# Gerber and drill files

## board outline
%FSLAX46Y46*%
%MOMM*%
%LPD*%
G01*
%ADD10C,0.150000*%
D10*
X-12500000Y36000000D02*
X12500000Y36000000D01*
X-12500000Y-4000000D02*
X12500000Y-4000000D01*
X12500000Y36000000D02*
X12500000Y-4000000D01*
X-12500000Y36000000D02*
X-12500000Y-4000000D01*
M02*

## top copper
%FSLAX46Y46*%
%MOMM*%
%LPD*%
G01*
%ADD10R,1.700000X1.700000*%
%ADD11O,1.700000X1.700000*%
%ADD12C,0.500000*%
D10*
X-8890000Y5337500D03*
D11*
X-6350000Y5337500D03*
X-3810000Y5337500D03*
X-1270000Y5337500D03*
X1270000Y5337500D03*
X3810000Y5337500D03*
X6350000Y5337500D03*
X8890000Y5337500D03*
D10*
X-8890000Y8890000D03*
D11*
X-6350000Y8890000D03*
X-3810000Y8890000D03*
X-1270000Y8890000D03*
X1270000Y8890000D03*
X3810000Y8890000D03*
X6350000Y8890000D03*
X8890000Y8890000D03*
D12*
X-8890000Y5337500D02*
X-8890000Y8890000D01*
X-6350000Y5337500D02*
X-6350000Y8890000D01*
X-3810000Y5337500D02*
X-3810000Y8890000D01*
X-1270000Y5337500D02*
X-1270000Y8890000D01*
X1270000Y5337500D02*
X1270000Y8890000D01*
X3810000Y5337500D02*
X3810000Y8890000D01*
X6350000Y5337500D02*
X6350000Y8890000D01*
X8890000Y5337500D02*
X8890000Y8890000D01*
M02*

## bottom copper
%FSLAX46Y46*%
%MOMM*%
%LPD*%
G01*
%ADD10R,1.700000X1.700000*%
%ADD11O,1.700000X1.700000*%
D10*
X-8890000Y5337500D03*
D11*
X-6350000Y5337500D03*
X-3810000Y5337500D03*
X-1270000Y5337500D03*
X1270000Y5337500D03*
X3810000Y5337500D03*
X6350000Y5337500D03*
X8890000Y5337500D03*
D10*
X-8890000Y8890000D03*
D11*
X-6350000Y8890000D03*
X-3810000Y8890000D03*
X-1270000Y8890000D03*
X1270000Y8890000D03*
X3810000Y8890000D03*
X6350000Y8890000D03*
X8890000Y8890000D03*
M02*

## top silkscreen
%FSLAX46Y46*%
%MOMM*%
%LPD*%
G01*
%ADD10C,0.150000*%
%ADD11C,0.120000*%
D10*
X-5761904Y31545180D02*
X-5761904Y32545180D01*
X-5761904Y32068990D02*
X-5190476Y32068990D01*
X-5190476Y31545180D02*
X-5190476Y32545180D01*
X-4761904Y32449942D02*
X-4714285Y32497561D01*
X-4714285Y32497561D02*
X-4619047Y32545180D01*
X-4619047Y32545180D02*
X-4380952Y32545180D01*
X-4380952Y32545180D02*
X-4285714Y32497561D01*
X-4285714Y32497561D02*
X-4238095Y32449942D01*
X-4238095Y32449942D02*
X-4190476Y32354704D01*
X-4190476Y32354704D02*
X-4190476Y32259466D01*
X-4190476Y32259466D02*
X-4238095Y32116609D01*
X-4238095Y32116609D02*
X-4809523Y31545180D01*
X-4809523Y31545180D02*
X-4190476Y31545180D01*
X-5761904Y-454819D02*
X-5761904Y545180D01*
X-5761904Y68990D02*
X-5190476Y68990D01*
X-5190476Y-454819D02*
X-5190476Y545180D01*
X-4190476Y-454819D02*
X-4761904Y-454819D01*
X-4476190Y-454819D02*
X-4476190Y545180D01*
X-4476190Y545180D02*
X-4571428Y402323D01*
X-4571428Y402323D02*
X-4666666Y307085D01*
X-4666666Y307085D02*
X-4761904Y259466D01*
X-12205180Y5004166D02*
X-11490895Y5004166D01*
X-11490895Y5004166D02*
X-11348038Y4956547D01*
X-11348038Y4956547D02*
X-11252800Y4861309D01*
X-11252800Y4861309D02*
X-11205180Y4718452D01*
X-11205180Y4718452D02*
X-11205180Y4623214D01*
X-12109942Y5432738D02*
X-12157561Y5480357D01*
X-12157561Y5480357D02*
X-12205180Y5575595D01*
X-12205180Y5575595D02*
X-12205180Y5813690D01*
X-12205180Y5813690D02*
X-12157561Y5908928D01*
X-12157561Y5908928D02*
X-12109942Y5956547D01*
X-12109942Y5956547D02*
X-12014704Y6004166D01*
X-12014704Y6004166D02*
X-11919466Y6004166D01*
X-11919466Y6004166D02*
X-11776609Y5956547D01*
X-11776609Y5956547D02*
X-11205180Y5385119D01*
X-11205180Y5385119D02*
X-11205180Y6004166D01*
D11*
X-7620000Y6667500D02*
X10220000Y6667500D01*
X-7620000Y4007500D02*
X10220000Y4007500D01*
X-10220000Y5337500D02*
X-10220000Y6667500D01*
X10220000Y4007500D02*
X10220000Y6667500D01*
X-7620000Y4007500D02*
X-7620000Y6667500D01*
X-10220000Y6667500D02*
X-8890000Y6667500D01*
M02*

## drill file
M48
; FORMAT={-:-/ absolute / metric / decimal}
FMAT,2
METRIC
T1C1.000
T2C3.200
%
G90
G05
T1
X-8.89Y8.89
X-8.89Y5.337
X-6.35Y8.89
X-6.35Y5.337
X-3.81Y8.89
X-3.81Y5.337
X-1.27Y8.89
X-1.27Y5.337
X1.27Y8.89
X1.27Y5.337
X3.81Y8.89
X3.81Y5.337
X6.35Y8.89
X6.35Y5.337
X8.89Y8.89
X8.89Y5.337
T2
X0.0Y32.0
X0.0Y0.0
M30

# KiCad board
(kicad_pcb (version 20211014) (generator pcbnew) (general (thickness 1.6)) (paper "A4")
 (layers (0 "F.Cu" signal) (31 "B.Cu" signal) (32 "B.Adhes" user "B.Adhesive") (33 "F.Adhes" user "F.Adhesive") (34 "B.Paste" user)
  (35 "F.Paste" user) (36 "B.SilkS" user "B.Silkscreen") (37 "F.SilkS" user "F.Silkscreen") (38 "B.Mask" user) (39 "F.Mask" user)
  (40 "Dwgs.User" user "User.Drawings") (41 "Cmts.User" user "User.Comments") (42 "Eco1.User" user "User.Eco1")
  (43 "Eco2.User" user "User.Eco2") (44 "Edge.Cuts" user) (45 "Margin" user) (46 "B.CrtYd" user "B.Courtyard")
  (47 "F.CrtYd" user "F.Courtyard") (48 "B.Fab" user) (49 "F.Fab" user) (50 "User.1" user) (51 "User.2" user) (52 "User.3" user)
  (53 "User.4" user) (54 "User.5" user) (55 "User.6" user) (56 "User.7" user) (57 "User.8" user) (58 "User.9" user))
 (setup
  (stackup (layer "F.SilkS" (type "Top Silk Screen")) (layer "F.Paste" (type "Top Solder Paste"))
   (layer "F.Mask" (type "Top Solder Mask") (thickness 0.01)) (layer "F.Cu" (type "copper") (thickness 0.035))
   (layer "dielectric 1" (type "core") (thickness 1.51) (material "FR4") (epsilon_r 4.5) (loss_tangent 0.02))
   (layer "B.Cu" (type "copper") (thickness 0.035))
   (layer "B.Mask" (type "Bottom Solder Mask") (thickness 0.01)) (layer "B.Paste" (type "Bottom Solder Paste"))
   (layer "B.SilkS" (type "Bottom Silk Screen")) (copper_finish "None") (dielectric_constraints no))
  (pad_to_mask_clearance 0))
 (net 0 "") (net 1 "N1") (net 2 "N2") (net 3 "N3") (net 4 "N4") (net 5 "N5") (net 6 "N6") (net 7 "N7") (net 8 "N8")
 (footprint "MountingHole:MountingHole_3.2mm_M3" (layer "F.Cu") (at 0 -32)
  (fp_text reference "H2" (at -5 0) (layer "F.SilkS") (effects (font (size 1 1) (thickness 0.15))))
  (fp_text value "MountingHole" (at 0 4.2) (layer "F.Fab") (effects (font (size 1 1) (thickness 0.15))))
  (pad "" np_thru_hole circle (at 0 0) (size 3.2 3.2) (drill 3.2) (layers *.Cu *.Mask)))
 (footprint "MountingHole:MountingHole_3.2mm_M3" (layer "F.Cu") (at 0 0)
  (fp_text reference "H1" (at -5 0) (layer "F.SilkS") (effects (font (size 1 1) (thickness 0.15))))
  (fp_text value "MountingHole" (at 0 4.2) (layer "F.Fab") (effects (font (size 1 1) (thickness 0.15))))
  (pad "" np_thru_hole circle (at 0 0) (size 3.2 3.2) (drill 3.2) (layers *.Cu *.Mask)))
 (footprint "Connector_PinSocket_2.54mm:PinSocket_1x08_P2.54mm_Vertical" (layer "F.Cu") (at -8.89 -5.3375 90)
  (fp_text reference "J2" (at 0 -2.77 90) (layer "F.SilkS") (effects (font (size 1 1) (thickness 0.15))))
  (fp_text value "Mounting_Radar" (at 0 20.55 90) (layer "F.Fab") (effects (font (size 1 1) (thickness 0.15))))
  (fp_line (start 1.33 1.27) (end 1.33 19.11) (layer "F.SilkS") (width 0.12))
  (fp_line (start -1.33 1.27) (end -1.33 19.11) (layer "F.SilkS") (width 0.12))
  (fp_line (start 0 -1.33) (end 1.33 -1.33) (layer "F.SilkS") (width 0.12))
  (fp_line (start -1.33 19.11) (end 1.33 19.11) (layer "F.SilkS") (width 0.12))
  (fp_line (start -1.33 1.27) (end 1.33 1.27) (layer "F.SilkS") (width 0.12))
  (fp_line (start 1.33 -1.33) (end 1.33 0) (layer "F.SilkS") (width 0.12))
  (pad "1" thru_hole rect (at 0 0 90) (size 1.7 1.7) (drill 1) (layers *.Cu *.Mask) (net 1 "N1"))
  (pad "2" thru_hole oval (at 0 2.54 90) (size 1.7 1.7) (drill 1) (layers *.Cu *.Mask) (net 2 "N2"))
  (pad "3" thru_hole oval (at 0 5.08 90) (size 1.7 1.7) (drill 1) (layers *.Cu *.Mask) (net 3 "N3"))
  (pad "4" thru_hole oval (at 0 7.62 90) (size 1.7 1.7) (drill 1) (layers *.Cu *.Mask) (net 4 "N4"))
  (pad "5" thru_hole oval (at 0 10.16 90) (size 1.7 1.7) (drill 1) (layers *.Cu *.Mask) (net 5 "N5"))
  (pad "6" thru_hole oval (at 0 12.7 90) (size 1.7 1.7) (drill 1) (layers *.Cu *.Mask) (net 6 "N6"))
  (pad "7" thru_hole oval (at 0 15.24 90) (size 1.7 1.7) (drill 1) (layers *.Cu *.Mask) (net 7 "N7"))
  (pad "8" thru_hole oval (at 0 17.78 90) (size 1.7 1.7) (drill 1) (layers *.Cu *.Mask) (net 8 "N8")))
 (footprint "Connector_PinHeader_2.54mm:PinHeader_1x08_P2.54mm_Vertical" (layer "B.Cu") (at -8.89 -8.89 -90)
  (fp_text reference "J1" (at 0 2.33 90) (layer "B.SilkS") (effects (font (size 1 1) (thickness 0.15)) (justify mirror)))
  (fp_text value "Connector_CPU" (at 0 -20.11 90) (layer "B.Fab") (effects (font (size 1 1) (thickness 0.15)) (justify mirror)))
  (pad "1" thru_hole rect (at 0 0 270) (size 1.7 1.7) (drill 1) (layers *.Cu *.Mask) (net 1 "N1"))
  (pad "2" thru_hole oval (at 0 -2.54 270) (size 1.7 1.7) (drill 1) (layers *.Cu *.Mask) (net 2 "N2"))
  (pad "3" thru_hole oval (at 0 -5.08 270) (size 1.7 1.7) (drill 1) (layers *.Cu *.Mask) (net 3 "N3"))
  (pad "4" thru_hole oval (at 0 -7.62 270) (size 1.7 1.7) (drill 1) (layers *.Cu *.Mask) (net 4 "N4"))
  (pad "5" thru_hole oval (at 0 -10.16 270) (size 1.7 1.7) (drill 1) (layers *.Cu *.Mask) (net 5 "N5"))
  (pad "6" thru_hole oval (at 0 -12.7 270) (size 1.7 1.7) (drill 1) (layers *.Cu *.Mask) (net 6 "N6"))
  (pad "7" thru_hole oval (at 0 -15.24 270) (size 1.7 1.7) (drill 1) (layers *.Cu *.Mask) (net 7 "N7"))
  (pad "8" thru_hole oval (at 0 -17.78 270) (size 1.7 1.7) (drill 1) (layers *.Cu *.Mask) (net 8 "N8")))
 (gr_line (start -12.5 -36) (end 12.5 -36) (layer "Edge.Cuts") (width 0.15))
 (gr_line (start -12.5 4) (end 12.5 4) (layer "Edge.Cuts") (width 0.15))
 (gr_line (start 12.5 -36) (end 12.5 4) (layer "Edge.Cuts") (width 0.15))
 (gr_line (start -12.5 -36) (end -12.5 4) (layer "Edge.Cuts") (width 0.15))
 (segment (start -8.89 -5.3375) (end -8.89 -8.89) (width 0.5) (layer "F.Cu") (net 1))
 (segment (start -6.35 -5.3375) (end -6.35 -8.89) (width 0.5) (layer "F.Cu") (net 2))
 (segment (start -3.81 -5.3375) (end -3.81 -8.89) (width 0.5) (layer "F.Cu") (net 3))
 (segment (start -1.27 -5.3375) (end -1.27 -8.89) (width 0.5) (layer "F.Cu") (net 4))
 (segment (start 1.27 -5.3375) (end 1.27 -8.89) (width 0.5) (layer "F.Cu") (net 5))
 (segment (start 3.81 -5.3375) (end 3.81 -8.89) (width 0.5) (layer "F.Cu") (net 6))
 (segment (start 6.35 -5.3375) (end 6.35 -8.89) (width 0.5) (layer "F.Cu") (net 7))
 (segment (start 8.89 -5.3375) (end 8.89 -8.89) (width 0.5) (layer "F.Cu") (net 8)))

